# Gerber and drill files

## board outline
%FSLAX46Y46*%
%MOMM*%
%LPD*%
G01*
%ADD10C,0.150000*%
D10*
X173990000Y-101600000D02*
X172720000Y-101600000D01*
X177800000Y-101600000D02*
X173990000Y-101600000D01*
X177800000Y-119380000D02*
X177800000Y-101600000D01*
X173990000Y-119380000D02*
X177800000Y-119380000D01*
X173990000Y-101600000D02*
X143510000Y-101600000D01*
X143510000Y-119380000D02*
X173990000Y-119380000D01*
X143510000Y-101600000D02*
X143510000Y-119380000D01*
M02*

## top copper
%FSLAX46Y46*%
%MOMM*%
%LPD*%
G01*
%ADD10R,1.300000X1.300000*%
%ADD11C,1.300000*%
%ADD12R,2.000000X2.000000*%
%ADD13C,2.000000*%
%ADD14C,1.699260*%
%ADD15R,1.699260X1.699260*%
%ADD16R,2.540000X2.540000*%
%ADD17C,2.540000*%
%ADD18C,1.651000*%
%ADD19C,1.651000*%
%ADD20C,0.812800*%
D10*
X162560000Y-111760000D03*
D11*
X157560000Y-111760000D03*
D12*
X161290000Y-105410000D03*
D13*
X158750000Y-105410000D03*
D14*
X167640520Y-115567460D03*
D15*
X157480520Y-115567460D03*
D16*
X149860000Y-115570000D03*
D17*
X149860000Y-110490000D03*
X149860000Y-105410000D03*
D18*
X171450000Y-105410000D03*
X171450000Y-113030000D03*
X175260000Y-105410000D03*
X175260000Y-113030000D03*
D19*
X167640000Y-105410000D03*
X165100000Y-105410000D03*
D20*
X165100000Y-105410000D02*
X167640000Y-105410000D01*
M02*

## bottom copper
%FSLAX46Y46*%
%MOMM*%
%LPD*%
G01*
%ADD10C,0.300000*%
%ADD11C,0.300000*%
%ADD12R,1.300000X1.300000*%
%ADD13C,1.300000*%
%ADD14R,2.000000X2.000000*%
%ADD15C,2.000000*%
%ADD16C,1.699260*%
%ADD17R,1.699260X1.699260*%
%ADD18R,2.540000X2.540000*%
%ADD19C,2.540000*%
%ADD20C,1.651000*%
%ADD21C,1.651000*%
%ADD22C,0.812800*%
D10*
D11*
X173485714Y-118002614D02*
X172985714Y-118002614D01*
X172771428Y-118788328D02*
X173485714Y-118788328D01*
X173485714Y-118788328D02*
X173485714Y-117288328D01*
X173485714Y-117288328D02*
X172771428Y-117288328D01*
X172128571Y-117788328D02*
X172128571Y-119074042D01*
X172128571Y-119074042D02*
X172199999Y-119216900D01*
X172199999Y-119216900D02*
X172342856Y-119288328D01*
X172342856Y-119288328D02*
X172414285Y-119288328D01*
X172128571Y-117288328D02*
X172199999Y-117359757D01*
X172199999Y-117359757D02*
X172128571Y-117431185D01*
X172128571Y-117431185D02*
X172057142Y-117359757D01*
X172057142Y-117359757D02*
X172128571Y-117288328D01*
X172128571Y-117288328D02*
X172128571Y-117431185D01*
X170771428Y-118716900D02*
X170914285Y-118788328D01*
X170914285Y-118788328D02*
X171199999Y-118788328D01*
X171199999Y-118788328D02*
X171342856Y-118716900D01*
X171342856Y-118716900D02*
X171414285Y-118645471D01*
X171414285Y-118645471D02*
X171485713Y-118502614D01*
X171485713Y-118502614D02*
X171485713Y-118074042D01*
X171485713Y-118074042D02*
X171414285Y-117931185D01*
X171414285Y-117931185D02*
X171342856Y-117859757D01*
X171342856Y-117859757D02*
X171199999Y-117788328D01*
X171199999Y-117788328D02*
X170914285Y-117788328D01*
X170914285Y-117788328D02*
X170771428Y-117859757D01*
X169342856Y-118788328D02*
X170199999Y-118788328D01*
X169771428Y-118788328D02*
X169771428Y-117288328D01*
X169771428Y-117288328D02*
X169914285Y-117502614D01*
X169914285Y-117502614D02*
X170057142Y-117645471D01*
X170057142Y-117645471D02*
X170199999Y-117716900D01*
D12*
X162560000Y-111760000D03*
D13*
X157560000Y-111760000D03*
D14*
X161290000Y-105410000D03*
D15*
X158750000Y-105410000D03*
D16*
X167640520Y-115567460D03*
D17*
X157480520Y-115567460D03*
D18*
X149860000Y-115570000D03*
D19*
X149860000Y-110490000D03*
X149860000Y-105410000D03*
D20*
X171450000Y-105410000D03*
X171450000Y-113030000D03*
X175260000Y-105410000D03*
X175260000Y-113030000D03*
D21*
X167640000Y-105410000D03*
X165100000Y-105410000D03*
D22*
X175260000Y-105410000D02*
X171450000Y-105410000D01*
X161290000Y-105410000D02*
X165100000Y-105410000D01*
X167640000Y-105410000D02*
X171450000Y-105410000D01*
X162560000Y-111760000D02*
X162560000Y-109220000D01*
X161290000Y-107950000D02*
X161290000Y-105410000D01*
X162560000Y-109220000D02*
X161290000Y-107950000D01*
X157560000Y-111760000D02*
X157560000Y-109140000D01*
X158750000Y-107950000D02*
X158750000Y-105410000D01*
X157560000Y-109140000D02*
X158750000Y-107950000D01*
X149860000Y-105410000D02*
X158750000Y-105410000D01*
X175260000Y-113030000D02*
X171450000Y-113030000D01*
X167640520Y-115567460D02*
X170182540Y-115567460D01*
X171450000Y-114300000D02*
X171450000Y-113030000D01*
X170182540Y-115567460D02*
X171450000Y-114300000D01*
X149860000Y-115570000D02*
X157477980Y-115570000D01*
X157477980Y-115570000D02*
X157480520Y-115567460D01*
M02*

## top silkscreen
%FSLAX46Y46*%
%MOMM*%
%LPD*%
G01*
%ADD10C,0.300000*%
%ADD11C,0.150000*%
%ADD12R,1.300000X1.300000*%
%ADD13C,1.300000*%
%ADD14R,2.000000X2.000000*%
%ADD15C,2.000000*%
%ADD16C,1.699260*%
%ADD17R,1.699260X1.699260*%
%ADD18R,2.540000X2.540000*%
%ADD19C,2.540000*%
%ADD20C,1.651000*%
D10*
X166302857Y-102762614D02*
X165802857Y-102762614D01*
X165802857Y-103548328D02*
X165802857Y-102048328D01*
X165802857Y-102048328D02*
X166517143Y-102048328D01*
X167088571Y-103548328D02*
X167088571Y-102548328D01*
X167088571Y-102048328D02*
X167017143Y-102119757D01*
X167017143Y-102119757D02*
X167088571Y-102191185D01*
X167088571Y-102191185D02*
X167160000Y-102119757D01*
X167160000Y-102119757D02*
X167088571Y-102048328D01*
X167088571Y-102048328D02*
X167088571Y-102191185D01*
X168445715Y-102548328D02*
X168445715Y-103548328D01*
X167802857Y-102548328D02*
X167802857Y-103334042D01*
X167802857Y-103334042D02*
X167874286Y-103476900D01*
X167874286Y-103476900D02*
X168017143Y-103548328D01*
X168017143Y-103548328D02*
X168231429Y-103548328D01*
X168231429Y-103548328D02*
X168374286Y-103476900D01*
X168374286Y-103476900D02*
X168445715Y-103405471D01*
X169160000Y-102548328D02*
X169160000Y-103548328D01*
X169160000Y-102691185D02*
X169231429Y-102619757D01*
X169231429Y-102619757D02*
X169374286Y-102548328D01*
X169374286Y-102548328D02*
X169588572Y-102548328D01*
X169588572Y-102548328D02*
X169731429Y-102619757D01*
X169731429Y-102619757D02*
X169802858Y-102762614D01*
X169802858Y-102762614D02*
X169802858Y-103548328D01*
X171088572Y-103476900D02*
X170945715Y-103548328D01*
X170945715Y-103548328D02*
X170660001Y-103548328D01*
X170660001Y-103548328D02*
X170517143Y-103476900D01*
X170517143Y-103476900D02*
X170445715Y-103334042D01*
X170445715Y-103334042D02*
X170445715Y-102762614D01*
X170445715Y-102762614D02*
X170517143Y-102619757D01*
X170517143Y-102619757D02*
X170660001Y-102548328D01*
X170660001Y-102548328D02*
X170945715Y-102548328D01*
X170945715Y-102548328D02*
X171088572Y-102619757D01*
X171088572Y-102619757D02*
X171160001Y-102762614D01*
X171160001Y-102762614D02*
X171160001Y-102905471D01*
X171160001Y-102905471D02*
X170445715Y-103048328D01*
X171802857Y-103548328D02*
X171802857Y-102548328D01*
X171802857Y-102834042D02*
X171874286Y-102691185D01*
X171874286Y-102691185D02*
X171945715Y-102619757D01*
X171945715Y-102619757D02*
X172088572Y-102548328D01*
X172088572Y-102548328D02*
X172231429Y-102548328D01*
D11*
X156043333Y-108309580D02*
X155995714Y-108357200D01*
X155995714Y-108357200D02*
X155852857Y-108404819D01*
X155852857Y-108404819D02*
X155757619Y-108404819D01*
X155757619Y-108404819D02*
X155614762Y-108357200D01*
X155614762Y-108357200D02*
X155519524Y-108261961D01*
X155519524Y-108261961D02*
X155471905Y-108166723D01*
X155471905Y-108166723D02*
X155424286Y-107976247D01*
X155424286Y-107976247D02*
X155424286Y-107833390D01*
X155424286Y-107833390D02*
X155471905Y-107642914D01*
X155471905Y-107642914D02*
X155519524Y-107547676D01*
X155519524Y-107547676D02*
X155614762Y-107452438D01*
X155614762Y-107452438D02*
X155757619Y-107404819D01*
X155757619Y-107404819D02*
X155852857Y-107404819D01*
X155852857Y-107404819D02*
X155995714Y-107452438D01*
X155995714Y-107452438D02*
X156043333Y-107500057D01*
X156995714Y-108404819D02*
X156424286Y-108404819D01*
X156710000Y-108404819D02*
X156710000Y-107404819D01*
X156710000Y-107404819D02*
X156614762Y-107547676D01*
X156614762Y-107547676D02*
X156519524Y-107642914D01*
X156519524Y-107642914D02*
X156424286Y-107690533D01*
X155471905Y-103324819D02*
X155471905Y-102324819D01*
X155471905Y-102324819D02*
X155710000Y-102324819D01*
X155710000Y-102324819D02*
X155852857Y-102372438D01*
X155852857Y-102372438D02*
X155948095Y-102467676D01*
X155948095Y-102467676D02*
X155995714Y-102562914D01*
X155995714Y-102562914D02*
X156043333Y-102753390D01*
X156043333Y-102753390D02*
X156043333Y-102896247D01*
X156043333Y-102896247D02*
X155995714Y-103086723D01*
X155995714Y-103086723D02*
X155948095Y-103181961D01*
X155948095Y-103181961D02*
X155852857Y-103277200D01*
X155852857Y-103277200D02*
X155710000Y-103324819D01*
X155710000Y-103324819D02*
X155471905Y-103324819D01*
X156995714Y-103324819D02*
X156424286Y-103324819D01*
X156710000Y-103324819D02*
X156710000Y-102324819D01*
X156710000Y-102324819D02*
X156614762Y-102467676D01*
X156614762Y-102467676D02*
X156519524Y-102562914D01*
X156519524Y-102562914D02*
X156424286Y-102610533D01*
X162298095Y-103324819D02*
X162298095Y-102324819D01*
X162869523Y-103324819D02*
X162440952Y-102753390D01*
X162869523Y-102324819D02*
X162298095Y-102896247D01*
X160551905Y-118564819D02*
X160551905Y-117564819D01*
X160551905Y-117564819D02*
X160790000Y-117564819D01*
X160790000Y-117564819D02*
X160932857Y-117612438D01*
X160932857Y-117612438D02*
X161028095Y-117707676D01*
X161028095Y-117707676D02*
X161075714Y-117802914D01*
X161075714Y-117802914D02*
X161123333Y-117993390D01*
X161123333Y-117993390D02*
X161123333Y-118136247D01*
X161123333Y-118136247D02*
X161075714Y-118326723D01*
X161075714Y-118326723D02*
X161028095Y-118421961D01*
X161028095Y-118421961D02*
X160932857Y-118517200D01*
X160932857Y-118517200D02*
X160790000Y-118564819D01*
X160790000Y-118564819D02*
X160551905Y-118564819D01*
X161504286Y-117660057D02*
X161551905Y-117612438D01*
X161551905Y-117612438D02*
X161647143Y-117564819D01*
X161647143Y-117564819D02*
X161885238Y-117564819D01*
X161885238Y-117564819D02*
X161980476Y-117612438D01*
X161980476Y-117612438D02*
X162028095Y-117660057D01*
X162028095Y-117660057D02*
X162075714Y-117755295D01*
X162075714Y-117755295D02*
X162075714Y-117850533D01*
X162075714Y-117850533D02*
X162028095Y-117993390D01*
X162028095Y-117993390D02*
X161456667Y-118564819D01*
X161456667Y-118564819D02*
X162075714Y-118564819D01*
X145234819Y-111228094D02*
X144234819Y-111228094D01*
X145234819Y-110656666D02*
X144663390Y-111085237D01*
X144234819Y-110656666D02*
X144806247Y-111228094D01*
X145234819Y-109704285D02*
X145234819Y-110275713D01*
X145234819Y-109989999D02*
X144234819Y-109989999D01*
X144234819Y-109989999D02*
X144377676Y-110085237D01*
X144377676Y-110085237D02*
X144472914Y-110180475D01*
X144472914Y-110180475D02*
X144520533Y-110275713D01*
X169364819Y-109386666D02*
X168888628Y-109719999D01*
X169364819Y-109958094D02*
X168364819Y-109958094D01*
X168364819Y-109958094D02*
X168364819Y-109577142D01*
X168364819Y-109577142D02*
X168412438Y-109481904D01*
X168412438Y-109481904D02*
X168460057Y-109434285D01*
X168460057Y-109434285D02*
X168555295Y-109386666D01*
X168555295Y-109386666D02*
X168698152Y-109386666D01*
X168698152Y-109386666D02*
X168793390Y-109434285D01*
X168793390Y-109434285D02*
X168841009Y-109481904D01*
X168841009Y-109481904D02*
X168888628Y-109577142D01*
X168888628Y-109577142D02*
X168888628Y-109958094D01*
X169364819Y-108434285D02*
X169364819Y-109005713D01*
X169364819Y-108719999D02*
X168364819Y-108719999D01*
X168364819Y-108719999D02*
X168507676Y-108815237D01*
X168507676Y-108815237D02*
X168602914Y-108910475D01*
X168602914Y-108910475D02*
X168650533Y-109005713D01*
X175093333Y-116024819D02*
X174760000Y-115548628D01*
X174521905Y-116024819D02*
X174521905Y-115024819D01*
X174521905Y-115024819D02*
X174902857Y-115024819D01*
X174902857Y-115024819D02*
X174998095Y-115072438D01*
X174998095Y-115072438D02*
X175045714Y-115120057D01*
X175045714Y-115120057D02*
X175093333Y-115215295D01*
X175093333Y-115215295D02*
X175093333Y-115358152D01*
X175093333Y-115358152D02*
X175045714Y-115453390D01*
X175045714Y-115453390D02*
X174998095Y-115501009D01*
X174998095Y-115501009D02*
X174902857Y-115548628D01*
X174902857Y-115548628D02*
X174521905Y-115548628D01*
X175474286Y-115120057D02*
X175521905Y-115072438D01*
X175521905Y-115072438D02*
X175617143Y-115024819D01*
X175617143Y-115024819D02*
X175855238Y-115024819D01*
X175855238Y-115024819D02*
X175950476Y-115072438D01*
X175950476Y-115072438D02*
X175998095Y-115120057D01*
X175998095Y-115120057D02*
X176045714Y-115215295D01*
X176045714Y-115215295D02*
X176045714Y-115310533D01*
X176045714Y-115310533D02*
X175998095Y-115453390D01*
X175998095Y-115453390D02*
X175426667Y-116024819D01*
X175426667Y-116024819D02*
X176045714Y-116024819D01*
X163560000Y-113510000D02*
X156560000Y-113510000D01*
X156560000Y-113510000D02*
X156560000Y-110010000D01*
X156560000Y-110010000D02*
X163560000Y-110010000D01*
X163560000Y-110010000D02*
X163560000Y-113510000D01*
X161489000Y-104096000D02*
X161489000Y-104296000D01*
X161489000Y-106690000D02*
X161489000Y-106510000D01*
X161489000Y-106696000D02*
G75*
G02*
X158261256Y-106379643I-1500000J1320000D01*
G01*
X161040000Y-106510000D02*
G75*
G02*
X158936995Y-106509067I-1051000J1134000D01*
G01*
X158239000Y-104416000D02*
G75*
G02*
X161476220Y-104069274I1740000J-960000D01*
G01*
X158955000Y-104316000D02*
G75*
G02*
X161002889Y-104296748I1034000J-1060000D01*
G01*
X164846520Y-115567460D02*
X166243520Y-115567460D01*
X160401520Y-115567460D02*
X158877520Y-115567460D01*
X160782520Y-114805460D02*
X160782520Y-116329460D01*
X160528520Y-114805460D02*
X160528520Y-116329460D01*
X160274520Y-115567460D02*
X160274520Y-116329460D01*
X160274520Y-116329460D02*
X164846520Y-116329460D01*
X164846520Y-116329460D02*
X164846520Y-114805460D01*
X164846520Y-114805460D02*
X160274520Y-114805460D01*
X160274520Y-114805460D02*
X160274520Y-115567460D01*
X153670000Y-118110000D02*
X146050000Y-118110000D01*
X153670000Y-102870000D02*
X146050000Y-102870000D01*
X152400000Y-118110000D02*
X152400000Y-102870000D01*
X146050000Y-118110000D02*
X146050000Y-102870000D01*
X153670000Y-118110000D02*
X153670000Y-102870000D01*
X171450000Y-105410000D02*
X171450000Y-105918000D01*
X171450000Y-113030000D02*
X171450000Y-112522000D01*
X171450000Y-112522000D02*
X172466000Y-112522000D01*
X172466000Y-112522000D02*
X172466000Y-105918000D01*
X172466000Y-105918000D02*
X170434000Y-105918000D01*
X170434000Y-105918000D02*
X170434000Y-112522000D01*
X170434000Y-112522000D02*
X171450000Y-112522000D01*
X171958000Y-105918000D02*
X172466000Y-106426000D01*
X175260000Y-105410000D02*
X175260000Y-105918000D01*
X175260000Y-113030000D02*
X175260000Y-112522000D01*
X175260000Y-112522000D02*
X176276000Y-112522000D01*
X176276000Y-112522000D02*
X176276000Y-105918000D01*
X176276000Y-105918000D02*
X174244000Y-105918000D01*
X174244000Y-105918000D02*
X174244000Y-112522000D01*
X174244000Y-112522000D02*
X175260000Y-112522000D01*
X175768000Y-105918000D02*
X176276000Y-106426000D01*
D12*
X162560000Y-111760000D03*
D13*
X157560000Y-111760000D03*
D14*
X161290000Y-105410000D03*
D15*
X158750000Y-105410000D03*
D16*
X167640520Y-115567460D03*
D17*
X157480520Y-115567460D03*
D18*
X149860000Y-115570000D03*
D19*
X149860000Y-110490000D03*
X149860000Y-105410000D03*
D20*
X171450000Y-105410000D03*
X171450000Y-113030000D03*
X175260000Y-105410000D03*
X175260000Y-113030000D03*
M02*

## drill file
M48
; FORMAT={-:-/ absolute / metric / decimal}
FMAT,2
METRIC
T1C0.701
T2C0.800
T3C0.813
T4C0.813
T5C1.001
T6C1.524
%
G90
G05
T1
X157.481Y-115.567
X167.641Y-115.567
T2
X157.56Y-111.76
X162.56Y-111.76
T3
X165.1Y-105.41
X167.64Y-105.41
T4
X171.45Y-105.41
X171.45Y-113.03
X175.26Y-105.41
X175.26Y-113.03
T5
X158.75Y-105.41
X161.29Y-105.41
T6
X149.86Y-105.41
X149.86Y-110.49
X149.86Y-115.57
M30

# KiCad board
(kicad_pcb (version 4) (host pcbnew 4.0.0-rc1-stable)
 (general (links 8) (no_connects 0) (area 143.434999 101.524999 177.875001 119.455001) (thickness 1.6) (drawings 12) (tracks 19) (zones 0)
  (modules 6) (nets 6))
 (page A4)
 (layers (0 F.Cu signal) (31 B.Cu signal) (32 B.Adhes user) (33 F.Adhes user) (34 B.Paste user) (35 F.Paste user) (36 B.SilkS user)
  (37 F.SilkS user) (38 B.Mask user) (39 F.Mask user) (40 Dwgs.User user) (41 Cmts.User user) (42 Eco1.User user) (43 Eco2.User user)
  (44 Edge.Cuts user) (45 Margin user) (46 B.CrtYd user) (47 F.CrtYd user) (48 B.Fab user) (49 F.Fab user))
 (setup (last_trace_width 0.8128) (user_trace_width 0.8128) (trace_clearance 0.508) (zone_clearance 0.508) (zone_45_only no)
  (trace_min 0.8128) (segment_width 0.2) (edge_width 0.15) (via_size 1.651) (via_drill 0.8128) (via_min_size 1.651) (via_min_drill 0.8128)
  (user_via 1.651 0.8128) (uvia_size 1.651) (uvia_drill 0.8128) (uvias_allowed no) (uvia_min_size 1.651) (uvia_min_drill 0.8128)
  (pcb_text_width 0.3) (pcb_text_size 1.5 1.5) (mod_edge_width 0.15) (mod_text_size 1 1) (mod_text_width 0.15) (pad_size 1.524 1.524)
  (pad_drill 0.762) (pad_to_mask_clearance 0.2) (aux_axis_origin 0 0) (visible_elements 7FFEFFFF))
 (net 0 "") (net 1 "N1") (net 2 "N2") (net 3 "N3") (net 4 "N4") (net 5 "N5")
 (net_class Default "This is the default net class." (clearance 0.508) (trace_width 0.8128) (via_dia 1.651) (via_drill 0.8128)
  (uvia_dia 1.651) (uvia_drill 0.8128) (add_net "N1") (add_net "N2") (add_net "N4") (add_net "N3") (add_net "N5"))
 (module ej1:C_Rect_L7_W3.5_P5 (layer F.Cu) (at 162.56 111.76 180)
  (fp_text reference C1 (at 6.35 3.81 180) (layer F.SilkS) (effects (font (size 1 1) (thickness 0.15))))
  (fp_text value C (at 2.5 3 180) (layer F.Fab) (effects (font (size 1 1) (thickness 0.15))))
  (fp_line (start -1 -1.75) (end 6 -1.75) (layer F.SilkS) (width 0.15))
  (fp_line (start 6 -1.75) (end 6 1.75) (layer F.SilkS) (width 0.15))
  (fp_line (start 6 1.75) (end -1 1.75) (layer F.SilkS) (width 0.15))
  (fp_line (start -1 1.75) (end -1 -1.75) (layer F.SilkS) (width 0.15))
  (pad 1 thru_hole rect (at 0 0 180) (size 1.3 1.3) (drill 0.8) (layers *.Cu *.Mask F.SilkS) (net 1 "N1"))
  (pad 2 thru_hole circle (at 5 0 180) (size 1.3 1.3) (drill 0.8) (layers *.Cu *.Mask F.SilkS) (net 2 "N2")))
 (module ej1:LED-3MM (layer F.Cu) (at 161.29 105.41 180)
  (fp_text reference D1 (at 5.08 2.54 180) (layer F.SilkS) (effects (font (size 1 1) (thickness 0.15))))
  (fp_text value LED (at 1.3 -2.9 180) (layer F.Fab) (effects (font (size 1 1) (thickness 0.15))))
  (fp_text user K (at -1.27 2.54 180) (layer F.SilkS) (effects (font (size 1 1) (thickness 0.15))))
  (fp_line (start -0.199 1.314) (end -0.199 1.114) (layer F.SilkS) (width 0.15))
  (fp_line (start -0.199 -1.28) (end -0.199 -1.1) (layer F.SilkS) (width 0.15))
  (fp_arc (start 1.301 0.034) (end -0.199 -1.286) (angle 108.5) (layer F.SilkS) (width 0.15))
  (fp_arc (start 1.301 0.034) (end 0.25 -1.1) (angle 85.7) (layer F.SilkS) (width 0.15))
  (fp_arc (start 1.311 0.034) (end 3.051 0.994) (angle 110) (layer F.SilkS) (width 0.15))
  (fp_arc (start 1.301 0.034) (end 2.335 1.094) (angle 87.5) (layer F.SilkS) (width 0.15))
  (pad 1 thru_hole rect (at 0 0 270) (size 2 2) (drill 1.00076) (layers *.Cu *.Mask F.SilkS) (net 1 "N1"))
  (pad 2 thru_hole circle (at 2.54 0 180) (size 2 2) (drill 1.00076) (layers *.Cu *.Mask F.SilkS) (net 2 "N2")))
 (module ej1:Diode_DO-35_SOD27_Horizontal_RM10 (layer F.Cu) (at 157.48 115.57)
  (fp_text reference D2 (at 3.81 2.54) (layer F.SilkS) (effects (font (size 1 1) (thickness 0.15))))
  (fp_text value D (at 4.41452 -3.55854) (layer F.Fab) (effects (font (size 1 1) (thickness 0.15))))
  (fp_line (start 7.36652 -0.00254) (end 8.76352 -0.00254) (layer F.SilkS) (width 0.15))
  (fp_line (start 2.92152 -0.00254) (end 1.39752 -0.00254) (layer F.SilkS) (width 0.15))
  (fp_line (start 3.30252 -0.76454) (end 3.30252 0.75946) (layer F.SilkS) (width 0.15))
  (fp_line (start 3.04852 -0.76454) (end 3.04852 0.75946) (layer F.SilkS) (width 0.15))
  (fp_line (start 2.79452 -0.00254) (end 2.79452 0.75946) (layer F.SilkS) (width 0.15))
  (fp_line (start 2.79452 0.75946) (end 7.36652 0.75946) (layer F.SilkS) (width 0.15))
  (fp_line (start 7.36652 0.75946) (end 7.36652 -0.76454) (layer F.SilkS) (width 0.15))
  (fp_line (start 7.36652 -0.76454) (end 2.79452 -0.76454) (layer F.SilkS) (width 0.15))
  (fp_line (start 2.79452 -0.76454) (end 2.79452 -0.00254) (layer F.SilkS) (width 0.15))
  (pad 2 thru_hole circle (at 10.16052 -0.00254 180) (size 1.69926 1.69926) (drill 0.70104) (layers *.Cu *.Mask F.SilkS) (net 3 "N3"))
  (pad 1 thru_hole rect (at 0.00052 -0.00254 180) (size 1.69926 1.69926) (drill 0.70104) (layers *.Cu *.Mask F.SilkS) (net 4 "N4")))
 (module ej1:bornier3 (layer F.Cu) (at 149.86 110.49 90)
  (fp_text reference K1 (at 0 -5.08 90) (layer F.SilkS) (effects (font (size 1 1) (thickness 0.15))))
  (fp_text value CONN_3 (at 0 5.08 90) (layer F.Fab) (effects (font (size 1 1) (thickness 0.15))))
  (fp_line (start -7.62 3.81) (end -7.62 -3.81) (layer F.SilkS) (width 0.15))
  (fp_line (start 7.62 3.81) (end 7.62 -3.81) (layer F.SilkS) (width 0.15))
  (fp_line (start -7.62 2.54) (end 7.62 2.54) (layer F.SilkS) (width 0.15))
  (fp_line (start -7.62 -3.81) (end 7.62 -3.81) (layer F.SilkS) (width 0.15))
  (fp_line (start -7.62 3.81) (end 7.62 3.81) (layer F.SilkS) (width 0.15))
  (pad 1 thru_hole rect (at -5.08 0 90) (size 2.54 2.54) (drill 1.524) (layers *.Cu *.Mask F.SilkS) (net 4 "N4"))
  (pad 2 thru_hole circle (at 0 0 90) (size 2.54 2.54) (drill 1.524) (layers *.Cu *.Mask F.SilkS) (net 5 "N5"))
  (pad 3 thru_hole circle (at 5.08 0 90) (size 2.54 2.54) (drill 1.524) (layers *.Cu *.Mask F.SilkS) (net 2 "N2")))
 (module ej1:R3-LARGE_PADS (layer F.Cu) (at 171.45 109.22 270)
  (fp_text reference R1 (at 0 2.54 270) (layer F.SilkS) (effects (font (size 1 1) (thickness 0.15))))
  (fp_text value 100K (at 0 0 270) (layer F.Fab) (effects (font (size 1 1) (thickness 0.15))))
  (fp_line (start -3.81 0) (end -3.302 0) (layer F.SilkS) (width 0.15))
  (fp_line (start 3.81 0) (end 3.302 0) (layer F.SilkS) (width 0.15))
  (fp_line (start 3.302 0) (end 3.302 -1.016) (layer F.SilkS) (width 0.15))
  (fp_line (start 3.302 -1.016) (end -3.302 -1.016) (layer F.SilkS) (width 0.15))
  (fp_line (start -3.302 -1.016) (end -3.302 1.016) (layer F.SilkS) (width 0.15))
  (fp_line (start -3.302 1.016) (end 3.302 1.016) (layer F.SilkS) (width 0.15))
  (fp_line (start 3.302 1.016) (end 3.302 0) (layer F.SilkS) (width 0.15))
  (fp_line (start -3.302 -0.508) (end -2.794 -1.016) (layer F.SilkS) (width 0.15))
  (pad 1 thru_hole circle (at -3.81 0 270) (size 1.651 1.651) (drill 0.8128) (layers *.Cu *.Mask F.SilkS) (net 1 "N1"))
  (pad 2 thru_hole circle (at 3.81 0 270) (size 1.651 1.651) (drill 0.8128) (layers *.Cu *.Mask F.SilkS) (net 3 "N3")))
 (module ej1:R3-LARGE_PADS (layer F.Cu) (at 175.26 109.22 270)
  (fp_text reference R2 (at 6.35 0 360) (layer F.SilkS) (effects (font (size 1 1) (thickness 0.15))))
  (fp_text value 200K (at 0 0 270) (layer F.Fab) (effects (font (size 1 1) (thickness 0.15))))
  (fp_line (start -3.81 0) (end -3.302 0) (layer F.SilkS) (width 0.15))
  (fp_line (start 3.81 0) (end 3.302 0) (layer F.SilkS) (width 0.15))
  (fp_line (start 3.302 0) (end 3.302 -1.016) (layer F.SilkS) (width 0.15))
  (fp_line (start 3.302 -1.016) (end -3.302 -1.016) (layer F.SilkS) (width 0.15))
  (fp_line (start -3.302 -1.016) (end -3.302 1.016) (layer F.SilkS) (width 0.15))
  (fp_line (start -3.302 1.016) (end 3.302 1.016) (layer F.SilkS) (width 0.15))
  (fp_line (start 3.302 1.016) (end 3.302 0) (layer F.SilkS) (width 0.15))
  (fp_line (start -3.302 -0.508) (end -2.794 -1.016) (layer F.SilkS) (width 0.15))
  (pad 1 thru_hole circle (at -3.81 0 270) (size 1.651 1.651) (drill 0.8128) (layers *.Cu *.Mask F.SilkS) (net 1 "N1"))
  (pad 2 thru_hole circle (at 3.81 0 270) (size 1.651 1.651) (drill 0.8128) (layers *.Cu *.Mask F.SilkS) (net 3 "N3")))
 (gr_line (start 173.99 101.6) (end 172.72 101.6) (angle 90) (layer Edge.Cuts) (width 0.15))
 (gr_line (start 177.8 101.6) (end 173.99 101.6) (angle 90) (layer Edge.Cuts) (width 0.15))
 (gr_line (start 177.8 119.38) (end 177.8 101.6) (angle 90) (layer Edge.Cuts) (width 0.15))
 (gr_line (start 173.99 119.38) (end 177.8 119.38) (angle 90) (layer Edge.Cuts) (width 0.15))
 (gr_line (start 173.99 101.6) (end 143.51 101.6) (angle 90) (layer Edge.Cuts) (width 0.15))
 (gr_line (start 143.51 119.38) (end 173.99 119.38) (angle 90) (layer Edge.Cuts) (width 0.15))
 (gr_line (start 143.51 101.6) (end 143.51 119.38) (angle 90) (layer Edge.Cuts) (width 0.15))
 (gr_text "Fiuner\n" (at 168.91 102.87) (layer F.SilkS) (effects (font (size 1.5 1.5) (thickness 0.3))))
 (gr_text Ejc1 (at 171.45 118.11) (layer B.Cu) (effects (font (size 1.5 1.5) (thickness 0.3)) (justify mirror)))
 (segment (start 175.26 105.41) (end 171.45 105.41) (width 0.8128) (layer B.Cu) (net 1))
 (segment (start 161.29 105.41) (end 165.1 105.41) (width 0.8128) (layer B.Cu) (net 1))
 (segment (start 167.64 105.41) (end 171.45 105.41) (width 0.8128) (layer B.Cu) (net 1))
 (segment (start 165.1 105.41) (end 167.64 105.41) (width 0.8128) (layer F.Cu) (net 1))
 (segment (start 162.56 111.76) (end 162.56 109.22) (width 0.8128) (layer B.Cu) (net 1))
 (segment (start 161.29 107.95) (end 161.29 105.41) (width 0.8128) (layer B.Cu) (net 1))
 (segment (start 162.56 109.22) (end 161.29 107.95) (width 0.8128) (layer B.Cu) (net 1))
 (segment (start 157.56 111.76) (end 157.56 109.14) (width 0.8128) (layer B.Cu) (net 2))
 (segment (start 158.75 107.95) (end 158.75 105.41) (width 0.8128) (layer B.Cu) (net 2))
 (segment (start 157.56 109.14) (end 158.75 107.95) (width 0.8128) (layer B.Cu) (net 2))
 (segment (start 149.86 105.41) (end 158.75 105.41) (width 0.8128) (layer B.Cu) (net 2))
 (segment (start 175.26 113.03) (end 171.45 113.03) (width 0.8128) (layer B.Cu) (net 3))
 (segment (start 167.64052 115.56746) (end 170.18254 115.56746) (width 0.8128) (layer B.Cu) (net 3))
 (segment (start 171.45 114.3) (end 171.45 113.03) (width 0.8128) (layer B.Cu) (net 3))
 (segment (start 170.18254 115.56746) (end 171.45 114.3) (width 0.8128) (layer B.Cu) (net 3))
 (segment (start 149.86 115.57) (end 157.47798 115.57) (width 0.8128) (layer B.Cu) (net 4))
 (segment (start 157.47798 115.57) (end 157.48052 115.56746) (width 0.8128) (layer B.Cu) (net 4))
 (via (at 167.64 105.41) (size 1.651) (drill 0.8128) (layers F.Cu B.Cu) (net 1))
 (via (at 165.1 105.41) (size 1.651) (drill 0.8128) (layers F.Cu B.Cu) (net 1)))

